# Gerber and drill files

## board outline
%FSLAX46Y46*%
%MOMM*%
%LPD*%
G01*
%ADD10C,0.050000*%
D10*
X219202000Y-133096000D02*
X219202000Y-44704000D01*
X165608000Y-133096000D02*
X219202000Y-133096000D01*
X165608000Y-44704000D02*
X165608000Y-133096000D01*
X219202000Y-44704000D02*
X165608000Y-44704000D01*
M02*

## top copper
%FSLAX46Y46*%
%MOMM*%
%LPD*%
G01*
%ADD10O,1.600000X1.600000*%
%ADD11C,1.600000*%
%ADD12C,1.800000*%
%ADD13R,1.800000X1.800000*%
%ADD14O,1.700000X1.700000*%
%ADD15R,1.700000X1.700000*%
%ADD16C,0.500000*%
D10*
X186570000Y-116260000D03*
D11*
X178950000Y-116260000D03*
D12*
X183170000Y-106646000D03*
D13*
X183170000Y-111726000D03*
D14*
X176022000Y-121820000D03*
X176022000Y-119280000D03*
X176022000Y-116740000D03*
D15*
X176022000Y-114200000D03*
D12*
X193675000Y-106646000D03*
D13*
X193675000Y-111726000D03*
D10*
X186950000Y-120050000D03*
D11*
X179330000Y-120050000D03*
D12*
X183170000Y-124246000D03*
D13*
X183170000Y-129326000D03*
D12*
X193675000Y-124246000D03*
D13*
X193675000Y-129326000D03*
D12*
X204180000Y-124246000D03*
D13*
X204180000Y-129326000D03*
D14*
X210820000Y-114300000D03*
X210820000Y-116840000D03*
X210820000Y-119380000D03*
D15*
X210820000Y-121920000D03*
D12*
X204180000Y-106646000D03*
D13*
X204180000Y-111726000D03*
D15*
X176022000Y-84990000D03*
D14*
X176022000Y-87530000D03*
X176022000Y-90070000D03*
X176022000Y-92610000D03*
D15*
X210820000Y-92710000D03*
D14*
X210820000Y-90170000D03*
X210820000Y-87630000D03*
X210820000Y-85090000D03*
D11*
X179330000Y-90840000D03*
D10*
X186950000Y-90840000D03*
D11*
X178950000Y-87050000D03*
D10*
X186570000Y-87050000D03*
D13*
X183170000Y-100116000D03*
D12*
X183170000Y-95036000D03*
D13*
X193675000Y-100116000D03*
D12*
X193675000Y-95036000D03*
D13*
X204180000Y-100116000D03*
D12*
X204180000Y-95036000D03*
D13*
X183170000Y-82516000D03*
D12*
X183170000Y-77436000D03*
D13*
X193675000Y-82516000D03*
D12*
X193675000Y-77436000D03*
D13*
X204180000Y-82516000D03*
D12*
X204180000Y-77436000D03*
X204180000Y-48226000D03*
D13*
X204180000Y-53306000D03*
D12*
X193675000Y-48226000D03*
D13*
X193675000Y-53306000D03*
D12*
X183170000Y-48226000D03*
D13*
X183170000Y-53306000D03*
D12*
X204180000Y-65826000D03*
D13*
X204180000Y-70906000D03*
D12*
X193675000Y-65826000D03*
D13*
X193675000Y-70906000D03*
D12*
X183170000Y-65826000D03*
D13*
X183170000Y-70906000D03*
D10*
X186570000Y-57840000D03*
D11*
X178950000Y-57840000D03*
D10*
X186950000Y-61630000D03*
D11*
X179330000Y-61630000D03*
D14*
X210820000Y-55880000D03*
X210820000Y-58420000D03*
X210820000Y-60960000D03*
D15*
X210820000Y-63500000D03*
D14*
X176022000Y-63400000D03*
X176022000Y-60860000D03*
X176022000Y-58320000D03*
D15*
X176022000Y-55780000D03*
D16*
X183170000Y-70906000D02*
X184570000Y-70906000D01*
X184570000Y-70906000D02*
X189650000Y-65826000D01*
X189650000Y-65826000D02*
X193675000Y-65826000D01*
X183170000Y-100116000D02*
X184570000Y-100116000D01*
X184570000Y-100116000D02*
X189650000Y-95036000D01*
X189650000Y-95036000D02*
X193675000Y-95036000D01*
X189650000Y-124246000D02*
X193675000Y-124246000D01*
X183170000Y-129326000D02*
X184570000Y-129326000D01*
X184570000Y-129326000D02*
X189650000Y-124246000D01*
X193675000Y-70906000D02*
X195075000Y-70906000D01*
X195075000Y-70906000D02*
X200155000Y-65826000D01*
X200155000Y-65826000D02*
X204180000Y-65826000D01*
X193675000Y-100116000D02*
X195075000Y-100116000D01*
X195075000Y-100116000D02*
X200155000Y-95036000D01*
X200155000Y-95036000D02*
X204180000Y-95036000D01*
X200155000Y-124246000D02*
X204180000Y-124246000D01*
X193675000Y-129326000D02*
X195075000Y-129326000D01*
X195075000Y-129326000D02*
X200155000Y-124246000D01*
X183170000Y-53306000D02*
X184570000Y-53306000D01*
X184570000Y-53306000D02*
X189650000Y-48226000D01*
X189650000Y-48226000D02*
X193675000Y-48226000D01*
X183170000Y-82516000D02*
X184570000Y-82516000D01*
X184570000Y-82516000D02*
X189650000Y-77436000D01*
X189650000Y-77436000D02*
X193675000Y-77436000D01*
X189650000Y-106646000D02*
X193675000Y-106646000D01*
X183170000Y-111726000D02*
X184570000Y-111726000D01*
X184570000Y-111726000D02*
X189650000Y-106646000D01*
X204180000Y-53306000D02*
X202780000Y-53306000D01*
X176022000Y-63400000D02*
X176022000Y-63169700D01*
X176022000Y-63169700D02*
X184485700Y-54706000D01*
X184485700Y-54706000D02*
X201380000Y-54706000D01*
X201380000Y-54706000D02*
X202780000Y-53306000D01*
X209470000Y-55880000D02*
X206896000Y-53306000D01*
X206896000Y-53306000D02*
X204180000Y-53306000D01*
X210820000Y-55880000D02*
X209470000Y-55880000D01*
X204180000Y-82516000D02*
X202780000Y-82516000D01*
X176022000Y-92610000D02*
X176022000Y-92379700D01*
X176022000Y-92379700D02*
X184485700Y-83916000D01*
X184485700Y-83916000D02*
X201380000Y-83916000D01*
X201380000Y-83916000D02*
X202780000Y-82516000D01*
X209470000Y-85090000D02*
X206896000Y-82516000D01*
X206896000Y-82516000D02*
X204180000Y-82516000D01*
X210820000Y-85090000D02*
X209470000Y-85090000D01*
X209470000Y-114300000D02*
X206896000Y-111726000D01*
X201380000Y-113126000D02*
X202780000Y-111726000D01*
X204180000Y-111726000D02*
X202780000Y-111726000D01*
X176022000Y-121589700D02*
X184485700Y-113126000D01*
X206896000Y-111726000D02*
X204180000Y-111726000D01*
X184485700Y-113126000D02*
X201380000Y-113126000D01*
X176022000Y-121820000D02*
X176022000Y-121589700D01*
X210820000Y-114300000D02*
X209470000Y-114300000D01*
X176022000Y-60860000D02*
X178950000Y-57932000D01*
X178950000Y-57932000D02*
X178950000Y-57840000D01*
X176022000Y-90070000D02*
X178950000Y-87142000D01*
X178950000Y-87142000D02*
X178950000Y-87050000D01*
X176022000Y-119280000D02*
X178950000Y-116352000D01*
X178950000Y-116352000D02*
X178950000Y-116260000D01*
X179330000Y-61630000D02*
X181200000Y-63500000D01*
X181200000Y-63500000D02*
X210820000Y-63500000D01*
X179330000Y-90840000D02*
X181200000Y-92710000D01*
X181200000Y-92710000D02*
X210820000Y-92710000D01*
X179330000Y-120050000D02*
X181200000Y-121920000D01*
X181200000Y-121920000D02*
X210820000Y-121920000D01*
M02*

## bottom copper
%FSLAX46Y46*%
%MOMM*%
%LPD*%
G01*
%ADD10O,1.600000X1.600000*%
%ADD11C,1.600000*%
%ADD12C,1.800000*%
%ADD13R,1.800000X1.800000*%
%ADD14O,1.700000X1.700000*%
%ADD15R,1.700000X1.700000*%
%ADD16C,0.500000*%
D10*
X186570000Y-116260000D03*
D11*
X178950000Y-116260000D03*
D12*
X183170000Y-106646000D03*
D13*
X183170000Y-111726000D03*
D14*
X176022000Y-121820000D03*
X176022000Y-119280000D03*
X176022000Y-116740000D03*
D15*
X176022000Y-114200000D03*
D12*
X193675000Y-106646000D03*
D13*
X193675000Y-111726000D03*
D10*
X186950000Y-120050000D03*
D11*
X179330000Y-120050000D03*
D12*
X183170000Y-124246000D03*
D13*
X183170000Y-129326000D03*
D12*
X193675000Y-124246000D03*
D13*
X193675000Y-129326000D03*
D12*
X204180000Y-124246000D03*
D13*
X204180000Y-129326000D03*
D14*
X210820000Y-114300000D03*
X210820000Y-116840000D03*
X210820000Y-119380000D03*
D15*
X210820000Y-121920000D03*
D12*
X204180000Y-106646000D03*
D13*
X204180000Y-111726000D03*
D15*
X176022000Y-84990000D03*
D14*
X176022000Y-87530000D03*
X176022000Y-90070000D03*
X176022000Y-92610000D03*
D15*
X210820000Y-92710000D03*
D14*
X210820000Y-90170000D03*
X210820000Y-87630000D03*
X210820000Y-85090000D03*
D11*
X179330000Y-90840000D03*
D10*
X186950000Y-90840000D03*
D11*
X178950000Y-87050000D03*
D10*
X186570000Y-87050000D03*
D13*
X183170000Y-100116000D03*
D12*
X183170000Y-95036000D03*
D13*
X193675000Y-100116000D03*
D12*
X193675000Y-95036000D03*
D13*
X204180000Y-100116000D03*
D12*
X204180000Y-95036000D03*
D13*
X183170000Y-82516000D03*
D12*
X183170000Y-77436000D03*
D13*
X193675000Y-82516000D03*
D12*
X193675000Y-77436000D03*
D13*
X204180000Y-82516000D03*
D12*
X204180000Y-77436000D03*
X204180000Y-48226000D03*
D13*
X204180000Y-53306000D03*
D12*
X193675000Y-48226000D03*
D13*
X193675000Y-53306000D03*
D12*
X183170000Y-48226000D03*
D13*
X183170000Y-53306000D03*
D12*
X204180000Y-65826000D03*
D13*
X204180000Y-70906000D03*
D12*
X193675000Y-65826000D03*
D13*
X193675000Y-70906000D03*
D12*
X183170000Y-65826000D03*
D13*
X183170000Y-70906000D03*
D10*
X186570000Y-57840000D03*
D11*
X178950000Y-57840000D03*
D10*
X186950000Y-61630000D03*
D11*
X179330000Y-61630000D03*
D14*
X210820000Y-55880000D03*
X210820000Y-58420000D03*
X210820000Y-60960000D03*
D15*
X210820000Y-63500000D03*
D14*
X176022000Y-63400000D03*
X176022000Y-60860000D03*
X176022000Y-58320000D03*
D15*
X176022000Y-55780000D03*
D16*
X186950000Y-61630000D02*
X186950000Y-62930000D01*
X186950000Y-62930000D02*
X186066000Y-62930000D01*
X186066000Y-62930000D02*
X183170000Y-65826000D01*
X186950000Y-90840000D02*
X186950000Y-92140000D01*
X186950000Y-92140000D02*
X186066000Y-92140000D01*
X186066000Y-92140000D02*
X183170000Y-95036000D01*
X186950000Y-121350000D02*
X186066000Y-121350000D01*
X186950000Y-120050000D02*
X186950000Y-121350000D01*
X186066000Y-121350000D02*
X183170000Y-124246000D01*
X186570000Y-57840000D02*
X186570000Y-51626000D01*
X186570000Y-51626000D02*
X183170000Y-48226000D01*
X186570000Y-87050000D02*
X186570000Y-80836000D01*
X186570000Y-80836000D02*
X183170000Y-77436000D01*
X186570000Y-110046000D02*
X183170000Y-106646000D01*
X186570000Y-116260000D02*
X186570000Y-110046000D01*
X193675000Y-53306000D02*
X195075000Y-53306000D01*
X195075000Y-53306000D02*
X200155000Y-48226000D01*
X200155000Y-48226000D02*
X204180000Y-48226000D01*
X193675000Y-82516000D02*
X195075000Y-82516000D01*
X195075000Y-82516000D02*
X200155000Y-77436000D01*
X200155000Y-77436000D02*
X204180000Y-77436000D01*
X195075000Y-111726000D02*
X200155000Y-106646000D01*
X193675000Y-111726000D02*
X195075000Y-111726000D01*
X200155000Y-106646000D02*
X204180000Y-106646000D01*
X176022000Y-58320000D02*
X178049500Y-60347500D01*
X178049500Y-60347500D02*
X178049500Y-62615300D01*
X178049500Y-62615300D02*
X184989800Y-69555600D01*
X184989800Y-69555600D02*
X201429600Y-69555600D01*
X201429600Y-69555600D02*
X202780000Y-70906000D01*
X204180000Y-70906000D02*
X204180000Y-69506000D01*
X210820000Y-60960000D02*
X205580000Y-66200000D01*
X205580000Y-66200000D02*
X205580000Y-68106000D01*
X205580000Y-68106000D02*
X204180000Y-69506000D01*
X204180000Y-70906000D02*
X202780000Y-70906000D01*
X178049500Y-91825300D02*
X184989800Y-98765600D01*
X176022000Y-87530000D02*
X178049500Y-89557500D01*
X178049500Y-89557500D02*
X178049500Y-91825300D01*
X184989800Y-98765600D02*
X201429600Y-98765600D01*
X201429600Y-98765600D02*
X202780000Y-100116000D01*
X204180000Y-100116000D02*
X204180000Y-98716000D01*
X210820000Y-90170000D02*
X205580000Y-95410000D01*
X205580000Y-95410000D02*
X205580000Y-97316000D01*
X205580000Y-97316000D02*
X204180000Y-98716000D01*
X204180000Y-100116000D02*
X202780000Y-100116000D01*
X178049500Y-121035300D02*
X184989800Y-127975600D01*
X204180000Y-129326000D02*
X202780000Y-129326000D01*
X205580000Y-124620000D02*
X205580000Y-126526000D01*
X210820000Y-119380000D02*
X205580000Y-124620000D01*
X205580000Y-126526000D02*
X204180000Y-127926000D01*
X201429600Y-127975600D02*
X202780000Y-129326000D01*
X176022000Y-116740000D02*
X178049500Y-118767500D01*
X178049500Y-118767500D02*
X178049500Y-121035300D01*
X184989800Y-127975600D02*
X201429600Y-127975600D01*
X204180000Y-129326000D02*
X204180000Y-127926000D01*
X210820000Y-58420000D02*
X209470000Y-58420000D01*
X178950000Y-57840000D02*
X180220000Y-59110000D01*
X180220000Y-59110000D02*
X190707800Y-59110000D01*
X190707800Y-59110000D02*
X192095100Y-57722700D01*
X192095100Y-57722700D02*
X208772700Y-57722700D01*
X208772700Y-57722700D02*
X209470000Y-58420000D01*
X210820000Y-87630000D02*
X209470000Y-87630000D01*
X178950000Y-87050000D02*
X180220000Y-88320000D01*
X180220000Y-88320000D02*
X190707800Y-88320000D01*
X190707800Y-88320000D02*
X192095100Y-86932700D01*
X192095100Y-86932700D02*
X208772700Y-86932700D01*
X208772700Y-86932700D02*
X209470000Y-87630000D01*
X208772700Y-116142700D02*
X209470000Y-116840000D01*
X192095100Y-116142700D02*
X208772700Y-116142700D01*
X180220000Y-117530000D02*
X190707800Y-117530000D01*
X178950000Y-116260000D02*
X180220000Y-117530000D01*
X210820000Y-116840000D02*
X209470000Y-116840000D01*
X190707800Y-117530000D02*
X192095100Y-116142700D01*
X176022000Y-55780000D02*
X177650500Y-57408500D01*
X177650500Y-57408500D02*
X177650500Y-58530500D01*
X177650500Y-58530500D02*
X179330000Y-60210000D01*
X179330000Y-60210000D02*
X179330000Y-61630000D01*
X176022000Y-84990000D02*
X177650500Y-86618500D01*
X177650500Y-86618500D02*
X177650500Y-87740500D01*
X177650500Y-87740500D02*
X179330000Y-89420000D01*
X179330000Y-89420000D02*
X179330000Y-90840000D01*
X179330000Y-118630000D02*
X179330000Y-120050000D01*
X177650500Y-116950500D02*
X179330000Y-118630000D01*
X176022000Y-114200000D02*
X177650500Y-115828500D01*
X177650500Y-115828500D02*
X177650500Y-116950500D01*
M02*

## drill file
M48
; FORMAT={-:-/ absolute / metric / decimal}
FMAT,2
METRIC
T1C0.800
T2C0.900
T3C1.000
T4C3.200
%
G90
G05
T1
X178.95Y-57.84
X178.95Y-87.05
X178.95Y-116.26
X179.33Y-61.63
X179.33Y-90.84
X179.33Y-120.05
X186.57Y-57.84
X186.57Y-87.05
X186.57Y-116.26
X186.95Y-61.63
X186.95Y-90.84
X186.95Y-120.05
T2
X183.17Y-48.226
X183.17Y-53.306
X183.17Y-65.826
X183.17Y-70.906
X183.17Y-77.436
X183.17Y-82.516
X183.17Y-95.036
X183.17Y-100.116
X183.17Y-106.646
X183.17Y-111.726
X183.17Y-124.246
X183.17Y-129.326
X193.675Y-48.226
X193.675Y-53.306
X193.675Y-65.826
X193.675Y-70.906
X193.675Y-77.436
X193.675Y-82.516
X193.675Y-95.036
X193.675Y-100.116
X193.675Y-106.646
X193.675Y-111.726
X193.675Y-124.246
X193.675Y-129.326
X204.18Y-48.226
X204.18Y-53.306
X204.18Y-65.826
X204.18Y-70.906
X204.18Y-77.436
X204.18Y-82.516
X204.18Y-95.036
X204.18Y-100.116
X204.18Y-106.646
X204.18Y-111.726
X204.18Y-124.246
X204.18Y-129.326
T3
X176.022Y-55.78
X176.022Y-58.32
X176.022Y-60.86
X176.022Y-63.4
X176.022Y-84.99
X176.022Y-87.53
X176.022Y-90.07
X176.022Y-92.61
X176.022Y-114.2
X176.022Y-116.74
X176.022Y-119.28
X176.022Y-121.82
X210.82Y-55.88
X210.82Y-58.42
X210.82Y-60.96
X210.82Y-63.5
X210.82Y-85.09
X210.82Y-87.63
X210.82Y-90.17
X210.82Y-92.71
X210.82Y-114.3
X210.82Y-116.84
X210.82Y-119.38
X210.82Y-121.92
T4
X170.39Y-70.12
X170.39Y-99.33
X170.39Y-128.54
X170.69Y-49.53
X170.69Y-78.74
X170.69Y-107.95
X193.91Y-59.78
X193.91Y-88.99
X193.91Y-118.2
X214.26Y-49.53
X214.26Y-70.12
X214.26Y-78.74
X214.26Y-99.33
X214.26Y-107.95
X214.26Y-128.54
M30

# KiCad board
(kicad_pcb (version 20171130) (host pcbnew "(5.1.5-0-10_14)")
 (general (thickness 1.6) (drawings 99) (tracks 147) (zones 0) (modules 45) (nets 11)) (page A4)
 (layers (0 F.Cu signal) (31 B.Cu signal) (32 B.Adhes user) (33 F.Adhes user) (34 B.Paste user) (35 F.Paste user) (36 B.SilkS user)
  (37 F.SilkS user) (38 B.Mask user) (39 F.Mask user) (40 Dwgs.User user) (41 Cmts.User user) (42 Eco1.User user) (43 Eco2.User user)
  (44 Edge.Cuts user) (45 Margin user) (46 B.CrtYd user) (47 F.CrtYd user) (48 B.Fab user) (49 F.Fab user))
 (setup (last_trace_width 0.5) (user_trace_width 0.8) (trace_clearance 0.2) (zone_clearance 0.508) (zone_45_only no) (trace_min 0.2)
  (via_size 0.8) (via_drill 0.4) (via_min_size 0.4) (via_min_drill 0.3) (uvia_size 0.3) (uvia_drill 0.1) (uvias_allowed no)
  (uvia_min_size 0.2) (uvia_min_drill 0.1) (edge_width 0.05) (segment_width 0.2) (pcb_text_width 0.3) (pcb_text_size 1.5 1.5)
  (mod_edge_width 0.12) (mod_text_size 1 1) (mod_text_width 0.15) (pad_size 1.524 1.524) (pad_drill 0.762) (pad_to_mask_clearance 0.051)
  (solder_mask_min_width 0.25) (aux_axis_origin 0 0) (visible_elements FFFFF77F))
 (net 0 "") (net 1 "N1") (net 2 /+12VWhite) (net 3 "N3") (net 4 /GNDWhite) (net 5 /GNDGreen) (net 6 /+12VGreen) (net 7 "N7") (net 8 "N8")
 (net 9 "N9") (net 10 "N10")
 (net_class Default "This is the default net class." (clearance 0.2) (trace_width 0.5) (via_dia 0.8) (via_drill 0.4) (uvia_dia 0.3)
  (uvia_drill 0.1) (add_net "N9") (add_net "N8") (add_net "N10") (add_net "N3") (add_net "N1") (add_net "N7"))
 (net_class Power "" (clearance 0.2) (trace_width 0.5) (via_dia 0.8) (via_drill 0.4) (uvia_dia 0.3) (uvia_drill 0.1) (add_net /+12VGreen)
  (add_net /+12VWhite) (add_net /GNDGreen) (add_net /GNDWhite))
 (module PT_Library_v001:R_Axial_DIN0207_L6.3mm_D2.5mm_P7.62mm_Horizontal (layer B.Cu) (at 178.95 116.26)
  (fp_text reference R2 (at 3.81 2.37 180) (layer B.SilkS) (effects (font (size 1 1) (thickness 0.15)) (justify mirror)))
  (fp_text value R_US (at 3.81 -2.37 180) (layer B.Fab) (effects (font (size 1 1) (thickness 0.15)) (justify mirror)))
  (pad 2 thru_hole oval (at 7.62 0) (size 1.6 1.6) (drill 0.8) (layers *.Cu *.Mask) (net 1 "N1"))
  (pad 1 thru_hole circle (at 0 0) (size 1.6 1.6) (drill 0.8) (layers *.Cu *.Mask) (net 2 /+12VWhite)))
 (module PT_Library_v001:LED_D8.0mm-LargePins (layer F.Cu) (at 183.17 111.726 90)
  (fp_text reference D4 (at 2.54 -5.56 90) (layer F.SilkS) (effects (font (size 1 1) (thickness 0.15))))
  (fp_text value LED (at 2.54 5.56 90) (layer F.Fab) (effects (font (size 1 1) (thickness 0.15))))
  (pad 2 thru_hole circle (at 5.08 0 90) (size 1.8 1.8) (drill 0.9) (layers *.Cu *.Mask) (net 1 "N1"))
  (pad 1 thru_hole rect (at 0 0 90) (size 1.8 1.8) (drill 0.9) (layers *.Cu *.Mask) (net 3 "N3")))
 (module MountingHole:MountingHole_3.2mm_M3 (layer F.Cu) (at 214.26 107.95)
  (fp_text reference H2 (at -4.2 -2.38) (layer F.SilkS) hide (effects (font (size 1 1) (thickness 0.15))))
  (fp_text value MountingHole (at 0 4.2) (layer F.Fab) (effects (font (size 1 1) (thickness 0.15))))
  (pad 1 np_thru_hole circle (at 0 0) (size 3.2 3.2) (drill 3.2) (layers *.Cu *.Mask)))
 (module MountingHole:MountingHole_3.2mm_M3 (layer F.Cu) (at 170.39 128.54)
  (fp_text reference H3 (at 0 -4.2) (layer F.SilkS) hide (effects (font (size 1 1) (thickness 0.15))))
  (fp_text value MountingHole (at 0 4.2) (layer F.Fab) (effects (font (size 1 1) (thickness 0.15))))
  (pad 1 np_thru_hole circle (at 0 0) (size 3.2 3.2) (drill 3.2) (layers *.Cu *.Mask)))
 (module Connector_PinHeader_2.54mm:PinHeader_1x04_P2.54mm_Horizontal (layer B.Cu) (at 176.022 114.2 180)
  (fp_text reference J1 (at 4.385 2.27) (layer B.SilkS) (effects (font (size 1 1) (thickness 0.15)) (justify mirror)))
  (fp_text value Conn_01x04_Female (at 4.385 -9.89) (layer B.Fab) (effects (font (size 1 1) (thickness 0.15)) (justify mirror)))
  (pad 4 thru_hole oval (at 0 -7.62 180) (size 1.7 1.7) (drill 1) (layers *.Cu *.Mask) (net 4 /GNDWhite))
  (pad 3 thru_hole oval (at 0 -5.08 180) (size 1.7 1.7) (drill 1) (layers *.Cu *.Mask) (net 2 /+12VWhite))
  (pad 2 thru_hole oval (at 0 -2.54 180) (size 1.7 1.7) (drill 1) (layers *.Cu *.Mask) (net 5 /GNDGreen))
  (pad 1 thru_hole rect (at 0 0 180) (size 1.7 1.7) (drill 1) (layers *.Cu *.Mask) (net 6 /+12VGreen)))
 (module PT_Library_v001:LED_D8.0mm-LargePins (layer F.Cu) (at 193.675 111.726 90)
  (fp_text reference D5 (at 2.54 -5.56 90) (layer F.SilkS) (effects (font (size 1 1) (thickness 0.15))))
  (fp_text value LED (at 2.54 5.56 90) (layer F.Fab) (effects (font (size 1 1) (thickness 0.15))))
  (pad 2 thru_hole circle (at 5.08 0 90) (size 1.8 1.8) (drill 0.9) (layers *.Cu *.Mask) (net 3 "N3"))
  (pad 1 thru_hole rect (at 0 0 90) (size 1.8 1.8) (drill 0.9) (layers *.Cu *.Mask) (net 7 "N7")))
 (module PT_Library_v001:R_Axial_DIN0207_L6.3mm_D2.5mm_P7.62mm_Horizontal (layer B.Cu) (at 179.33 120.05)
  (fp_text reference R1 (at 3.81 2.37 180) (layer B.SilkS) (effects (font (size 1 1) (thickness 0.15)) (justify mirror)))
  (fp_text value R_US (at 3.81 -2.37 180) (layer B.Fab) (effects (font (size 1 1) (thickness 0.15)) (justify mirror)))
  (pad 2 thru_hole oval (at 7.62 0) (size 1.6 1.6) (drill 0.8) (layers *.Cu *.Mask) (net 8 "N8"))
  (pad 1 thru_hole circle (at 0 0) (size 1.6 1.6) (drill 0.8) (layers *.Cu *.Mask) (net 6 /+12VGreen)))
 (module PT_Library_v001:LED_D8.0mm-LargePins (layer F.Cu) (at 183.17 129.326 90)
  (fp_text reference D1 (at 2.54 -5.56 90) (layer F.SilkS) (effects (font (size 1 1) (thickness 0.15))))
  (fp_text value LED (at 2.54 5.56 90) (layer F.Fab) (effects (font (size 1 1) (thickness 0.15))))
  (pad 2 thru_hole circle (at 5.08 0 90) (size 1.8 1.8) (drill 0.9) (layers *.Cu *.Mask) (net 8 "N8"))
  (pad 1 thru_hole rect (at 0 0 90) (size 1.8 1.8) (drill 0.9) (layers *.Cu *.Mask) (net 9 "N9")))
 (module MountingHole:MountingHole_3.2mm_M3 (layer F.Cu) (at 170.69 107.95)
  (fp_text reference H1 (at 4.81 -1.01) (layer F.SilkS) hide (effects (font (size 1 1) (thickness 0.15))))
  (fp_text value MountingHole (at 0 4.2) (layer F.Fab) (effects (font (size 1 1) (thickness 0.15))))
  (pad 1 np_thru_hole circle (at 0 0) (size 3.2 3.2) (drill 3.2) (layers *.Cu *.Mask)))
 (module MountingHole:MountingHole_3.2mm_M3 (layer F.Cu) (at 193.91 118.2)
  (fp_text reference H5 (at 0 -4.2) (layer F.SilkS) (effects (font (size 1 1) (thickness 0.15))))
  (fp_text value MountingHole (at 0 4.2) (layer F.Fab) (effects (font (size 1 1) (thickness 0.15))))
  (pad 1 np_thru_hole circle (at 0 0) (size 3.2 3.2) (drill 3.2) (layers *.Cu *.Mask)))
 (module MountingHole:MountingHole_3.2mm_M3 (layer F.Cu) (at 214.26 128.54)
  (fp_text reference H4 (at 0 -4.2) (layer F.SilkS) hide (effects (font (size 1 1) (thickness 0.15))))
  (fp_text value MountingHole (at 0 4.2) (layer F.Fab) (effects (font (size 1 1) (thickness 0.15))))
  (pad 1 np_thru_hole circle (at 0 0) (size 3.2 3.2) (drill 3.2) (layers *.Cu *.Mask)))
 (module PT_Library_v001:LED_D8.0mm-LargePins (layer F.Cu) (at 193.675 129.326 90)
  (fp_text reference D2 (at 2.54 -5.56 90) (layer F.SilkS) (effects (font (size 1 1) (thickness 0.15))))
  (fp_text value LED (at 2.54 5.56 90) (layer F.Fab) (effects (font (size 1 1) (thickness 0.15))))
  (pad 2 thru_hole circle (at 5.08 0 90) (size 1.8 1.8) (drill 0.9) (layers *.Cu *.Mask) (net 9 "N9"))
  (pad 1 thru_hole rect (at 0 0 90) (size 1.8 1.8) (drill 0.9) (layers *.Cu *.Mask) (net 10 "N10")))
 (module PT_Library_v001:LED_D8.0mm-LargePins (layer F.Cu) (at 204.18 129.326 90)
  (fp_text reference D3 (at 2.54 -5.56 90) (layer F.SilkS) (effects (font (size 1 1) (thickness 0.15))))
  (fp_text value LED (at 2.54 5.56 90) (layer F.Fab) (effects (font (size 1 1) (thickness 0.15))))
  (pad 2 thru_hole circle (at 5.08 0 90) (size 1.8 1.8) (drill 0.9) (layers *.Cu *.Mask) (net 10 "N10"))
  (pad 1 thru_hole rect (at 0 0 90) (size 1.8 1.8) (drill 0.9) (layers *.Cu *.Mask) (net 5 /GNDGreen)))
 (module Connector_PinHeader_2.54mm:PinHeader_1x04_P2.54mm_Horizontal (layer B.Cu) (at 210.82 121.92)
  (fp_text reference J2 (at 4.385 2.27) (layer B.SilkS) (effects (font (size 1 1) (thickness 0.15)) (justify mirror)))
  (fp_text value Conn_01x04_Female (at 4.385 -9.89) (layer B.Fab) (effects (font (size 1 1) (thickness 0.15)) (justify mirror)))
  (pad 4 thru_hole oval (at 0 -7.62) (size 1.7 1.7) (drill 1) (layers *.Cu *.Mask) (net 4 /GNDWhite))
  (pad 3 thru_hole oval (at 0 -5.08) (size 1.7 1.7) (drill 1) (layers *.Cu *.Mask) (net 2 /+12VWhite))
  (pad 2 thru_hole oval (at 0 -2.54) (size 1.7 1.7) (drill 1) (layers *.Cu *.Mask) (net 5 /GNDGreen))
  (pad 1 thru_hole rect (at 0 0) (size 1.7 1.7) (drill 1) (layers *.Cu *.Mask) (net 6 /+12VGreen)))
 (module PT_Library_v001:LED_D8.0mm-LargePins (layer F.Cu) (at 204.18 111.726 90)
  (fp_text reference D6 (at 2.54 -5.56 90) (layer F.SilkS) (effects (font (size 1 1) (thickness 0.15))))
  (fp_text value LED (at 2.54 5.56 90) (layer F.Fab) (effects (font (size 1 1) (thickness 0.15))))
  (pad 2 thru_hole circle (at 5.08 0 90) (size 1.8 1.8) (drill 0.9) (layers *.Cu *.Mask) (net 7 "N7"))
  (pad 1 thru_hole rect (at 0 0 90) (size 1.8 1.8) (drill 0.9) (layers *.Cu *.Mask) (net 4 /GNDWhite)))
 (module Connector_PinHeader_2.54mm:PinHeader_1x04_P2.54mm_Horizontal (layer B.Cu) (at 176.022 84.99 180)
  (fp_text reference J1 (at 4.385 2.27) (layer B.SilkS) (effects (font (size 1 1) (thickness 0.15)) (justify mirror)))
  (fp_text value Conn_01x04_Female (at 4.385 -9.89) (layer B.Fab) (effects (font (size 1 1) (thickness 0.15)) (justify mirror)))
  (pad 1 thru_hole rect (at 0 0 180) (size 1.7 1.7) (drill 1) (layers *.Cu *.Mask) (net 6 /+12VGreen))
  (pad 2 thru_hole oval (at 0 -2.54 180) (size 1.7 1.7) (drill 1) (layers *.Cu *.Mask) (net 5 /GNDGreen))
  (pad 3 thru_hole oval (at 0 -5.08 180) (size 1.7 1.7) (drill 1) (layers *.Cu *.Mask) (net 2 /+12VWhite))
  (pad 4 thru_hole oval (at 0 -7.62 180) (size 1.7 1.7) (drill 1) (layers *.Cu *.Mask) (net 4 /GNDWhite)))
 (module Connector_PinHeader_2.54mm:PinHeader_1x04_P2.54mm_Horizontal (layer B.Cu) (at 210.82 92.71)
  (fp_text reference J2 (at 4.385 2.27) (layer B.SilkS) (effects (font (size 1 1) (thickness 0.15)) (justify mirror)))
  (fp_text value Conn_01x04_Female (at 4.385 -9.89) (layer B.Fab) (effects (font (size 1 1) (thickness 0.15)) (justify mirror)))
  (pad 1 thru_hole rect (at 0 0) (size 1.7 1.7) (drill 1) (layers *.Cu *.Mask) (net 6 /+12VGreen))
  (pad 2 thru_hole oval (at 0 -2.54) (size 1.7 1.7) (drill 1) (layers *.Cu *.Mask) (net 5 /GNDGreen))
  (pad 3 thru_hole oval (at 0 -5.08) (size 1.7 1.7) (drill 1) (layers *.Cu *.Mask) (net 2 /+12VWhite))
  (pad 4 thru_hole oval (at 0 -7.62) (size 1.7 1.7) (drill 1) (layers *.Cu *.Mask) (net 4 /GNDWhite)))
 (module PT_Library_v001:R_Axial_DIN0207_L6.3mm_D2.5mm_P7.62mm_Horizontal (layer B.Cu) (at 179.33 90.84)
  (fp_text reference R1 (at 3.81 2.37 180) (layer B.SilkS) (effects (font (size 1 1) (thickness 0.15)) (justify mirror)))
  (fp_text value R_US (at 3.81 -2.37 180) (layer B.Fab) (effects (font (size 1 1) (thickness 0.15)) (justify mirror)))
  (pad 1 thru_hole circle (at 0 0) (size 1.6 1.6) (drill 0.8) (layers *.Cu *.Mask) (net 6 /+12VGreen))
  (pad 2 thru_hole oval (at 7.62 0) (size 1.6 1.6) (drill 0.8) (layers *.Cu *.Mask) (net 8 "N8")))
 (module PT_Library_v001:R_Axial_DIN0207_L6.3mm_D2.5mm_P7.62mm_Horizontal (layer B.Cu) (at 178.95 87.05)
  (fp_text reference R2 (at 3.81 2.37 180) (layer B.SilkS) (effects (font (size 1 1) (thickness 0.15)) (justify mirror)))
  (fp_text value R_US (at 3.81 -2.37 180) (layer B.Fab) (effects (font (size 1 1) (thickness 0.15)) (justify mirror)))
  (pad 1 thru_hole circle (at 0 0) (size 1.6 1.6) (drill 0.8) (layers *.Cu *.Mask) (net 2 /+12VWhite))
  (pad 2 thru_hole oval (at 7.62 0) (size 1.6 1.6) (drill 0.8) (layers *.Cu *.Mask) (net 1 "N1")))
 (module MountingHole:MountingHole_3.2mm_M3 (layer F.Cu) (at 170.69 78.74)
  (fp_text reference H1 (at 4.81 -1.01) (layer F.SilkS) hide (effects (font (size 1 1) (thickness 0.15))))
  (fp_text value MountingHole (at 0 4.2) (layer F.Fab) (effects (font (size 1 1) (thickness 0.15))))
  (pad 1 np_thru_hole circle (at 0 0) (size 3.2 3.2) (drill 3.2) (layers *.Cu *.Mask)))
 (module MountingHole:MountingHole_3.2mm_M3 (layer F.Cu) (at 214.26 78.74)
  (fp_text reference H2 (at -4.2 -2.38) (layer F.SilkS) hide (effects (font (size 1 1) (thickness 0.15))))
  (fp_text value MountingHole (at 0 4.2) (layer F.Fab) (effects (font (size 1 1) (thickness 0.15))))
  (pad 1 np_thru_hole circle (at 0 0) (size 3.2 3.2) (drill 3.2) (layers *.Cu *.Mask)))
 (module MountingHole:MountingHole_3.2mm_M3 (layer F.Cu) (at 170.39 99.33)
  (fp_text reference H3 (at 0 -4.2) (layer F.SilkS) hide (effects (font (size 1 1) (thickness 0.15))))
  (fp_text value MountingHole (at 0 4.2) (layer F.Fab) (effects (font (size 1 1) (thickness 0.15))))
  (pad 1 np_thru_hole circle (at 0 0) (size 3.2 3.2) (drill 3.2) (layers *.Cu *.Mask)))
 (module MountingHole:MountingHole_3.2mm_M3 (layer F.Cu) (at 214.26 99.33)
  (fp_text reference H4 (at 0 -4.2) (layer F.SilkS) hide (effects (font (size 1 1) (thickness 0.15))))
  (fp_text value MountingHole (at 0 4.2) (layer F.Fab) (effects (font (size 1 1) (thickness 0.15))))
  (pad 1 np_thru_hole circle (at 0 0) (size 3.2 3.2) (drill 3.2) (layers *.Cu *.Mask)))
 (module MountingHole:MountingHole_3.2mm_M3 (layer F.Cu) (at 193.91 88.99)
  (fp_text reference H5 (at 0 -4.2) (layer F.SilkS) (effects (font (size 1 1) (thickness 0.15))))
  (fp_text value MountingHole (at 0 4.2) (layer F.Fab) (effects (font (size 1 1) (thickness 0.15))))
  (pad 1 np_thru_hole circle (at 0 0) (size 3.2 3.2) (drill 3.2) (layers *.Cu *.Mask)))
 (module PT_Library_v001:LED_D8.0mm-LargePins (layer F.Cu) (at 183.17 100.116 90)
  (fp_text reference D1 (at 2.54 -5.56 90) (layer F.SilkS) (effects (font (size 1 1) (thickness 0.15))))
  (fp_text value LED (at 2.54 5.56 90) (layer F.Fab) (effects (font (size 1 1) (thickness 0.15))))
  (pad 1 thru_hole rect (at 0 0 90) (size 1.8 1.8) (drill 0.9) (layers *.Cu *.Mask) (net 9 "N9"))
  (pad 2 thru_hole circle (at 5.08 0 90) (size 1.8 1.8) (drill 0.9) (layers *.Cu *.Mask) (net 8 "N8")))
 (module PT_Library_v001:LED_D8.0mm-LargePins (layer F.Cu) (at 193.675 100.116 90)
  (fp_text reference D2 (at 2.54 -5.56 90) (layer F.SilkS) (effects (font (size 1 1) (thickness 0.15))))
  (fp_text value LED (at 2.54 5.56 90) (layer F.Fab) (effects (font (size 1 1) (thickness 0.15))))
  (pad 1 thru_hole rect (at 0 0 90) (size 1.8 1.8) (drill 0.9) (layers *.Cu *.Mask) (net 10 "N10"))
  (pad 2 thru_hole circle (at 5.08 0 90) (size 1.8 1.8) (drill 0.9) (layers *.Cu *.Mask) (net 9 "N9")))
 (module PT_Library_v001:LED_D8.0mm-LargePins (layer F.Cu) (at 204.18 100.116 90)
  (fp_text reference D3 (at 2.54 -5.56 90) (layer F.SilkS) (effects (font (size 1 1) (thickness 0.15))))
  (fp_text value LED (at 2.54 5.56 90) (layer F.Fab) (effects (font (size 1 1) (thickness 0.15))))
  (pad 1 thru_hole rect (at 0 0 90) (size 1.8 1.8) (drill 0.9) (layers *.Cu *.Mask) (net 5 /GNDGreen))
  (pad 2 thru_hole circle (at 5.08 0 90) (size 1.8 1.8) (drill 0.9) (layers *.Cu *.Mask) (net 10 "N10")))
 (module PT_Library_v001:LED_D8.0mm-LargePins (layer F.Cu) (at 183.17 82.516 90)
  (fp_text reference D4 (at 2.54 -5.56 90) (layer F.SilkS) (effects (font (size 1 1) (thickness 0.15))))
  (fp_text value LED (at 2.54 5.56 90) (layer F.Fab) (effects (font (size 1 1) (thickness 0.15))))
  (pad 1 thru_hole rect (at 0 0 90) (size 1.8 1.8) (drill 0.9) (layers *.Cu *.Mask) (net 3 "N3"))
  (pad 2 thru_hole circle (at 5.08 0 90) (size 1.8 1.8) (drill 0.9) (layers *.Cu *.Mask) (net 1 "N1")))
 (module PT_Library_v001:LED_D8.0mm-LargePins (layer F.Cu) (at 193.675 82.516 90)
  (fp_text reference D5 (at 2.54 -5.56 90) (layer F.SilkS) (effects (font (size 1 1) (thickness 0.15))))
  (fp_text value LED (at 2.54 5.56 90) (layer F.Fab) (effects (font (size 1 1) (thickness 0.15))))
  (pad 1 thru_hole rect (at 0 0 90) (size 1.8 1.8) (drill 0.9) (layers *.Cu *.Mask) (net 7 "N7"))
  (pad 2 thru_hole circle (at 5.08 0 90) (size 1.8 1.8) (drill 0.9) (layers *.Cu *.Mask) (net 3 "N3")))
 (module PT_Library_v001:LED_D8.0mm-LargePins (layer F.Cu) (at 204.18 82.516 90)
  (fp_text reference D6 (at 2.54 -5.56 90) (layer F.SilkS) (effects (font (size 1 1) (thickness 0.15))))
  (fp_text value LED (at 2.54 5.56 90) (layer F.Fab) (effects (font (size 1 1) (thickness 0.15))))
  (pad 1 thru_hole rect (at 0 0 90) (size 1.8 1.8) (drill 0.9) (layers *.Cu *.Mask) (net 4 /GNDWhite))
  (pad 2 thru_hole circle (at 5.08 0 90) (size 1.8 1.8) (drill 0.9) (layers *.Cu *.Mask) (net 7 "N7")))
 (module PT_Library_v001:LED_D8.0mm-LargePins (layer F.Cu) (at 204.18 53.306 90)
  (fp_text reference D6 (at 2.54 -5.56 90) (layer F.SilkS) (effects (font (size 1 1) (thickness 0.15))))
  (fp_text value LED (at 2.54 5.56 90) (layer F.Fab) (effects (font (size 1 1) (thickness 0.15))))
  (pad 2 thru_hole circle (at 5.08 0 90) (size 1.8 1.8) (drill 0.9) (layers *.Cu *.Mask) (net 7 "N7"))
  (pad 1 thru_hole rect (at 0 0 90) (size 1.8 1.8) (drill 0.9) (layers *.Cu *.Mask) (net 4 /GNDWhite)))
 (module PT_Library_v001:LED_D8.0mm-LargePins (layer F.Cu) (at 193.675 53.306 90)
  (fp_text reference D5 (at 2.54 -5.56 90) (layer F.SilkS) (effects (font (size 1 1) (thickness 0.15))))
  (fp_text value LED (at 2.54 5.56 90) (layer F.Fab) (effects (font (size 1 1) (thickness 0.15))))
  (pad 2 thru_hole circle (at 5.08 0 90) (size 1.8 1.8) (drill 0.9) (layers *.Cu *.Mask) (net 3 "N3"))
  (pad 1 thru_hole rect (at 0 0 90) (size 1.8 1.8) (drill 0.9) (layers *.Cu *.Mask) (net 7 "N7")))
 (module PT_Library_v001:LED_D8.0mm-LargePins (layer F.Cu) (at 183.17 53.306 90)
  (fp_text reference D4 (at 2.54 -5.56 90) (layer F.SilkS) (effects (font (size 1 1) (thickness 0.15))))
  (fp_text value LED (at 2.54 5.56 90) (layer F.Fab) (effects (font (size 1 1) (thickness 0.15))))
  (pad 2 thru_hole circle (at 5.08 0 90) (size 1.8 1.8) (drill 0.9) (layers *.Cu *.Mask) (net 1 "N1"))
  (pad 1 thru_hole rect (at 0 0 90) (size 1.8 1.8) (drill 0.9) (layers *.Cu *.Mask) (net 3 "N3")))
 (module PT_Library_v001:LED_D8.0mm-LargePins (layer F.Cu) (at 204.18 70.906 90)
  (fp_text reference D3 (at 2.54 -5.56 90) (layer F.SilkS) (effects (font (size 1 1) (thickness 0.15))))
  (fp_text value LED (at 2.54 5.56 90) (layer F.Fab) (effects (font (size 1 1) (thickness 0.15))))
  (pad 2 thru_hole circle (at 5.08 0 90) (size 1.8 1.8) (drill 0.9) (layers *.Cu *.Mask) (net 10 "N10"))
  (pad 1 thru_hole rect (at 0 0 90) (size 1.8 1.8) (drill 0.9) (layers *.Cu *.Mask) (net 5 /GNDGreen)))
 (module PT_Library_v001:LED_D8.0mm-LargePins (layer F.Cu) (at 193.675 70.906 90)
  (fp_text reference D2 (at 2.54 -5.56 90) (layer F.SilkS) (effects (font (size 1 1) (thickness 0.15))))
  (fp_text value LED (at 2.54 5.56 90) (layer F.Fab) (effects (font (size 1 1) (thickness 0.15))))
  (pad 2 thru_hole circle (at 5.08 0 90) (size 1.8 1.8) (drill 0.9) (layers *.Cu *.Mask) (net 9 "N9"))
  (pad 1 thru_hole rect (at 0 0 90) (size 1.8 1.8) (drill 0.9) (layers *.Cu *.Mask) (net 10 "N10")))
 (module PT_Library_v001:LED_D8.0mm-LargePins (layer F.Cu) (at 183.17 70.906 90)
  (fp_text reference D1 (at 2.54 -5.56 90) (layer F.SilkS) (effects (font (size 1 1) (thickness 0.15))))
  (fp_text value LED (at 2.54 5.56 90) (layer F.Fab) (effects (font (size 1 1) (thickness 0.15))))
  (pad 2 thru_hole circle (at 5.08 0 90) (size 1.8 1.8) (drill 0.9) (layers *.Cu *.Mask) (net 8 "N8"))
  (pad 1 thru_hole rect (at 0 0 90) (size 1.8 1.8) (drill 0.9) (layers *.Cu *.Mask) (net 9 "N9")))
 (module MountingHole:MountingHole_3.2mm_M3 (layer F.Cu) (at 193.91 59.78)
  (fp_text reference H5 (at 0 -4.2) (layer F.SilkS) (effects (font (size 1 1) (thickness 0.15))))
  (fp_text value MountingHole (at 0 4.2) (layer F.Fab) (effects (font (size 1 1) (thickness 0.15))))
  (pad 1 np_thru_hole circle (at 0 0) (size 3.2 3.2) (drill 3.2) (layers *.Cu *.Mask)))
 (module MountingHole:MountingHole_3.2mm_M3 (layer F.Cu) (at 214.26 70.12)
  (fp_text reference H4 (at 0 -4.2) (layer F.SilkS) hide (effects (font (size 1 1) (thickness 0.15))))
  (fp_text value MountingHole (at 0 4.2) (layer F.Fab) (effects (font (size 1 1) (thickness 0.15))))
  (pad 1 np_thru_hole circle (at 0 0) (size 3.2 3.2) (drill 3.2) (layers *.Cu *.Mask)))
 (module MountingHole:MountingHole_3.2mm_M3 (layer F.Cu) (at 170.39 70.12)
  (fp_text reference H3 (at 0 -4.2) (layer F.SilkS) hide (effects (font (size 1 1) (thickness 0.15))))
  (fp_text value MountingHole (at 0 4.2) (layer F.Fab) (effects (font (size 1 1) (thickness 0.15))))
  (pad 1 np_thru_hole circle (at 0 0) (size 3.2 3.2) (drill 3.2) (layers *.Cu *.Mask)))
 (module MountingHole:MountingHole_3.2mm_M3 (layer F.Cu) (at 214.26 49.53)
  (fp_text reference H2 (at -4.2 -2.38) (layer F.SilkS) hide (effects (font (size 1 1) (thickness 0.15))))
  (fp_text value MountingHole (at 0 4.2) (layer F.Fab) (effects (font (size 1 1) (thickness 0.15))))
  (pad 1 np_thru_hole circle (at 0 0) (size 3.2 3.2) (drill 3.2) (layers *.Cu *.Mask)))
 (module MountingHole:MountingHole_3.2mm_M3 (layer F.Cu) (at 170.69 49.53)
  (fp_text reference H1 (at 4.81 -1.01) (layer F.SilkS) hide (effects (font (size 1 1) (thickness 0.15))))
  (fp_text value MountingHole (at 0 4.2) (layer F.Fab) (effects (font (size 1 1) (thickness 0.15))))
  (pad 1 np_thru_hole circle (at 0 0) (size 3.2 3.2) (drill 3.2) (layers *.Cu *.Mask)))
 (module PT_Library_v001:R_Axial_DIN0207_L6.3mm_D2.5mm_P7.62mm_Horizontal (layer B.Cu) (at 178.95 57.84)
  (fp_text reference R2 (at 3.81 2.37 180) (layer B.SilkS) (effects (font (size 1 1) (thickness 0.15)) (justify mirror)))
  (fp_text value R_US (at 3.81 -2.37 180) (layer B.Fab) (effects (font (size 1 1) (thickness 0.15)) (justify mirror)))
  (pad 2 thru_hole oval (at 7.62 0) (size 1.6 1.6) (drill 0.8) (layers *.Cu *.Mask) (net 1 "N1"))
  (pad 1 thru_hole circle (at 0 0) (size 1.6 1.6) (drill 0.8) (layers *.Cu *.Mask) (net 2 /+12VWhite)))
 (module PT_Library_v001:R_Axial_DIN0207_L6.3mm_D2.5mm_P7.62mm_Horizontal (layer B.Cu) (at 179.33 61.63)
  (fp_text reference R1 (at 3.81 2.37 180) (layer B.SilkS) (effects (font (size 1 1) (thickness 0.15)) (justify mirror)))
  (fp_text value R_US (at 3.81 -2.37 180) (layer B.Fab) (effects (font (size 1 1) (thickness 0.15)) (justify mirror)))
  (pad 2 thru_hole oval (at 7.62 0) (size 1.6 1.6) (drill 0.8) (layers *.Cu *.Mask) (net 8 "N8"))
  (pad 1 thru_hole circle (at 0 0) (size 1.6 1.6) (drill 0.8) (layers *.Cu *.Mask) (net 6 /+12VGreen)))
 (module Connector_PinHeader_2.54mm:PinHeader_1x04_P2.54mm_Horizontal (layer B.Cu) (at 210.82 63.5)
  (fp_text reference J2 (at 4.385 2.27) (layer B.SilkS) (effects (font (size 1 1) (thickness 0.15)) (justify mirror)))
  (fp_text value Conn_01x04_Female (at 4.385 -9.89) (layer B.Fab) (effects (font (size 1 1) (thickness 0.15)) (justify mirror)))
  (pad 4 thru_hole oval (at 0 -7.62) (size 1.7 1.7) (drill 1) (layers *.Cu *.Mask) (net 4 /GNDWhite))
  (pad 3 thru_hole oval (at 0 -5.08) (size 1.7 1.7) (drill 1) (layers *.Cu *.Mask) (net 2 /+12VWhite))
  (pad 2 thru_hole oval (at 0 -2.54) (size 1.7 1.7) (drill 1) (layers *.Cu *.Mask) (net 5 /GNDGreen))
  (pad 1 thru_hole rect (at 0 0) (size 1.7 1.7) (drill 1) (layers *.Cu *.Mask) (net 6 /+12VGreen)))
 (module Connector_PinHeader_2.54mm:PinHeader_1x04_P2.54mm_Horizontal (layer B.Cu) (at 176.022 55.78 180)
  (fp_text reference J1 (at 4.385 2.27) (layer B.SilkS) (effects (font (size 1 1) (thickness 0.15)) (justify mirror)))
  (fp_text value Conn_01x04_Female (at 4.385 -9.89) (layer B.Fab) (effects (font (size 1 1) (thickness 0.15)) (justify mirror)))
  (pad 4 thru_hole oval (at 0 -7.62 180) (size 1.7 1.7) (drill 1) (layers *.Cu *.Mask) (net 4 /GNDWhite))
  (pad 3 thru_hole oval (at 0 -5.08 180) (size 1.7 1.7) (drill 1) (layers *.Cu *.Mask) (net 2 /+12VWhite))
  (pad 2 thru_hole oval (at 0 -2.54 180) (size 1.7 1.7) (drill 1) (layers *.Cu *.Mask) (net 5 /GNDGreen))
  (pad 1 thru_hole rect (at 0 0 180) (size 1.7 1.7) (drill 1) (layers *.Cu *.Mask) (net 6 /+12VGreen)))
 (gr_line (start 219.202 133.096) (end 219.202 44.704) (layer Edge.Cuts) (width 0.05))
 (gr_line (start 165.608 133.096) (end 219.202 133.096) (layer Edge.Cuts) (width 0.05))
 (gr_line (start 165.608 44.704) (end 165.608 133.096) (layer Edge.Cuts) (width 0.05))
 (gr_line (start 219.202 44.704) (end 165.608 44.704) (layer Edge.Cuts) (width 0.05))
 (segment (start 183.17 70.906) (end 184.57 70.906) (width 0.5) (layer F.Cu) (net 9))
 (segment (start 184.57 70.906) (end 189.65 65.826) (width 0.5) (layer F.Cu) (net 9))
 (segment (start 189.65 65.826) (end 193.675 65.826) (width 0.5) (layer F.Cu) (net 9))
 (segment (start 183.17 100.116) (end 184.57 100.116) (width 0.5) (layer F.Cu) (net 9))
 (segment (start 184.57 100.116) (end 189.65 95.036) (width 0.5) (layer F.Cu) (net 9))
 (segment (start 189.65 95.036) (end 193.675 95.036) (width 0.5) (layer F.Cu) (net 9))
 (segment (start 189.65 124.246) (end 193.675 124.246) (width 0.5) (layer F.Cu) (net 9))
 (segment (start 183.17 129.326) (end 184.57 129.326) (width 0.5) (layer F.Cu) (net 9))
 (segment (start 184.57 129.326) (end 189.65 124.246) (width 0.5) (layer F.Cu) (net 9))
 (segment (start 186.95 61.63) (end 186.95 62.93) (width 0.5) (layer B.Cu) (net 8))
 (segment (start 186.95 62.93) (end 186.066 62.93) (width 0.5) (layer B.Cu) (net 8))
 (segment (start 186.066 62.93) (end 183.17 65.826) (width 0.5) (layer B.Cu) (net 8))
 (segment (start 186.95 90.84) (end 186.95 92.14) (width 0.5) (layer B.Cu) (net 8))
 (segment (start 186.95 92.14) (end 186.066 92.14) (width 0.5) (layer B.Cu) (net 8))
 (segment (start 186.066 92.14) (end 183.17 95.036) (width 0.5) (layer B.Cu) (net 8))
 (segment (start 186.95 121.35) (end 186.066 121.35) (width 0.5) (layer B.Cu) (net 8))
 (segment (start 186.95 120.05) (end 186.95 121.35) (width 0.5) (layer B.Cu) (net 8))
 (segment (start 186.066 121.35) (end 183.17 124.246) (width 0.5) (layer B.Cu) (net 8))
 (segment (start 193.675 70.906) (end 195.075 70.906) (width 0.5) (layer F.Cu) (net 10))
 (segment (start 195.075 70.906) (end 200.155 65.826) (width 0.5) (layer F.Cu) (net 10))
 (segment (start 200.155 65.826) (end 204.18 65.826) (width 0.5) (layer F.Cu) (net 10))
 (segment (start 193.675 100.116) (end 195.075 100.116) (width 0.5) (layer F.Cu) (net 10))
 (segment (start 195.075 100.116) (end 200.155 95.036) (width 0.5) (layer F.Cu) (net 10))
 (segment (start 200.155 95.036) (end 204.18 95.036) (width 0.5) (layer F.Cu) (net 10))
 (segment (start 200.155 124.246) (end 204.18 124.246) (width 0.5) (layer F.Cu) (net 10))
 (segment (start 193.675 129.326) (end 195.075 129.326) (width 0.5) (layer F.Cu) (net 10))
 (segment (start 195.075 129.326) (end 200.155 124.246) (width 0.5) (layer F.Cu) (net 10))
 (segment (start 186.57 57.84) (end 186.57 51.626) (width 0.5) (layer B.Cu) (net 1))
 (segment (start 186.57 51.626) (end 183.17 48.226) (width 0.5) (layer B.Cu) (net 1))
 (segment (start 186.57 87.05) (end 186.57 80.836) (width 0.5) (layer B.Cu) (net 1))
 (segment (start 186.57 80.836) (end 183.17 77.436) (width 0.5) (layer B.Cu) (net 1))
 (segment (start 186.57 110.046) (end 183.17 106.646) (width 0.5) (layer B.Cu) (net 1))
 (segment (start 186.57 116.26) (end 186.57 110.046) (width 0.5) (layer B.Cu) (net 1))
 (segment (start 183.17 53.306) (end 184.57 53.306) (width 0.5) (layer F.Cu) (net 3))
 (segment (start 184.57 53.306) (end 189.65 48.226) (width 0.5) (layer F.Cu) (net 3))
 (segment (start 189.65 48.226) (end 193.675 48.226) (width 0.5) (layer F.Cu) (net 3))
 (segment (start 183.17 82.516) (end 184.57 82.516) (width 0.5) (layer F.Cu) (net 3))
 (segment (start 184.57 82.516) (end 189.65 77.436) (width 0.5) (layer F.Cu) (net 3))
 (segment (start 189.65 77.436) (end 193.675 77.436) (width 0.5) (layer F.Cu) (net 3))
 (segment (start 189.65 106.646) (end 193.675 106.646) (width 0.5) (layer F.Cu) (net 3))
 (segment (start 183.17 111.726) (end 184.57 111.726) (width 0.5) (layer F.Cu) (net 3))
 (segment (start 184.57 111.726) (end 189.65 106.646) (width 0.5) (layer F.Cu) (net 3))
 (segment (start 193.675 53.306) (end 195.075 53.306) (width 0.5) (layer B.Cu) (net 7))
 (segment (start 195.075 53.306) (end 200.155 48.226) (width 0.5) (layer B.Cu) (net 7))
 (segment (start 200.155 48.226) (end 204.18 48.226) (width 0.5) (layer B.Cu) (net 7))
 (segment (start 193.675 82.516) (end 195.075 82.516) (width 0.5) (layer B.Cu) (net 7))
 (segment (start 195.075 82.516) (end 200.155 77.436) (width 0.5) (layer B.Cu) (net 7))
 (segment (start 200.155 77.436) (end 204.18 77.436) (width 0.5) (layer B.Cu) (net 7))
 (segment (start 195.075 111.726) (end 200.155 106.646) (width 0.5) (layer B.Cu) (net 7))
 (segment (start 193.675 111.726) (end 195.075 111.726) (width 0.5) (layer B.Cu) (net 7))
 (segment (start 200.155 106.646) (end 204.18 106.646) (width 0.5) (layer B.Cu) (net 7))
 (segment (start 176.022 58.32) (end 178.0495 60.3475) (width 0.5) (layer B.Cu) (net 5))
 (segment (start 178.0495 60.3475) (end 178.0495 62.6153) (width 0.5) (layer B.Cu) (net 5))
 (segment (start 178.0495 62.6153) (end 184.9898 69.5556) (width 0.5) (layer B.Cu) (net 5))
 (segment (start 184.9898 69.5556) (end 201.4296 69.5556) (width 0.5) (layer B.Cu) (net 5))
 (segment (start 201.4296 69.5556) (end 202.78 70.906) (width 0.5) (layer B.Cu) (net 5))
 (segment (start 204.18 70.906) (end 204.18 69.506) (width 0.5) (layer B.Cu) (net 5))
 (segment (start 210.82 60.96) (end 205.58 66.2) (width 0.5) (layer B.Cu) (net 5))
 (segment (start 205.58 66.2) (end 205.58 68.106) (width 0.5) (layer B.Cu) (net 5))
 (segment (start 205.58 68.106) (end 204.18 69.506) (width 0.5) (layer B.Cu) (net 5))
 (segment (start 204.18 70.906) (end 202.78 70.906) (width 0.5) (layer B.Cu) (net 5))
 (segment (start 178.0495 91.8253) (end 184.9898 98.7656) (width 0.5) (layer B.Cu) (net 5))
 (segment (start 176.022 87.53) (end 178.0495 89.5575) (width 0.5) (layer B.Cu) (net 5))
 (segment (start 178.0495 89.5575) (end 178.0495 91.8253) (width 0.5) (layer B.Cu) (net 5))
 (segment (start 184.9898 98.7656) (end 201.4296 98.7656) (width 0.5) (layer B.Cu) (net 5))
 (segment (start 201.4296 98.7656) (end 202.78 100.116) (width 0.5) (layer B.Cu) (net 5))
 (segment (start 204.18 100.116) (end 204.18 98.716) (width 0.5) (layer B.Cu) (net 5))
 (segment (start 210.82 90.17) (end 205.58 95.41) (width 0.5) (layer B.Cu) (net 5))
 (segment (start 205.58 95.41) (end 205.58 97.316) (width 0.5) (layer B.Cu) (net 5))
 (segment (start 205.58 97.316) (end 204.18 98.716) (width 0.5) (layer B.Cu) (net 5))
 (segment (start 204.18 100.116) (end 202.78 100.116) (width 0.5) (layer B.Cu) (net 5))
 (segment (start 178.0495 121.0353) (end 184.9898 127.9756) (width 0.5) (layer B.Cu) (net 5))
 (segment (start 204.18 129.326) (end 202.78 129.326) (width 0.5) (layer B.Cu) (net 5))
 (segment (start 205.58 124.62) (end 205.58 126.526) (width 0.5) (layer B.Cu) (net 5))
 (segment (start 210.82 119.38) (end 205.58 124.62) (width 0.5) (layer B.Cu) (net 5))
 (segment (start 205.58 126.526) (end 204.18 127.926) (width 0.5) (layer B.Cu) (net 5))
 (segment (start 201.4296 127.9756) (end 202.78 129.326) (width 0.5) (layer B.Cu) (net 5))
 (segment (start 176.022 116.74) (end 178.0495 118.7675) (width 0.5) (layer B.Cu) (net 5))
 (segment (start 178.0495 118.7675) (end 178.0495 121.0353) (width 0.5) (layer B.Cu) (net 5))
 (segment (start 184.9898 127.9756) (end 201.4296 127.9756) (width 0.5) (layer B.Cu) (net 5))
 (segment (start 204.18 129.326) (end 204.18 127.926) (width 0.5) (layer B.Cu) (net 5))
 (segment (start 204.18 53.306) (end 202.78 53.306) (width 0.5) (layer F.Cu) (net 4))
 (segment (start 176.022 63.4) (end 176.022 63.1697) (width 0.5) (layer F.Cu) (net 4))
 (segment (start 176.022 63.1697) (end 184.4857 54.706) (width 0.5) (layer F.Cu) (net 4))
 (segment (start 184.4857 54.706) (end 201.38 54.706) (width 0.5) (layer F.Cu) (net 4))
 (segment (start 201.38 54.706) (end 202.78 53.306) (width 0.5) (layer F.Cu) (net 4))
 (segment (start 209.47 55.88) (end 206.896 53.306) (width 0.5) (layer F.Cu) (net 4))
 (segment (start 206.896 53.306) (end 204.18 53.306) (width 0.5) (layer F.Cu) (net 4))
 (segment (start 210.82 55.88) (end 209.47 55.88) (width 0.5) (layer F.Cu) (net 4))
 (segment (start 204.18 82.516) (end 202.78 82.516) (width 0.5) (layer F.Cu) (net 4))
 (segment (start 176.022 92.61) (end 176.022 92.3797) (width 0.5) (layer F.Cu) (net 4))
 (segment (start 176.022 92.3797) (end 184.4857 83.916) (width 0.5) (layer F.Cu) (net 4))
 (segment (start 184.4857 83.916) (end 201.38 83.916) (width 0.5) (layer F.Cu) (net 4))
 (segment (start 201.38 83.916) (end 202.78 82.516) (width 0.5) (layer F.Cu) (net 4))
 (segment (start 209.47 85.09) (end 206.896 82.516) (width 0.5) (layer F.Cu) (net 4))
 (segment (start 206.896 82.516) (end 204.18 82.516) (width 0.5) (layer F.Cu) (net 4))
 (segment (start 210.82 85.09) (end 209.47 85.09) (width 0.5) (layer F.Cu) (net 4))
 (segment (start 209.47 114.3) (end 206.896 111.726) (width 0.5) (layer F.Cu) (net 4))
 (segment (start 201.38 113.126) (end 202.78 111.726) (width 0.5) (layer F.Cu) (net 4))
 (segment (start 204.18 111.726) (end 202.78 111.726) (width 0.5) (layer F.Cu) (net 4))
 (segment (start 176.022 121.5897) (end 184.4857 113.126) (width 0.5) (layer F.Cu) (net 4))
 (segment (start 206.896 111.726) (end 204.18 111.726) (width 0.5) (layer F.Cu) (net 4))
 (segment (start 184.4857 113.126) (end 201.38 113.126) (width 0.5) (layer F.Cu) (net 4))
 (segment (start 176.022 121.82) (end 176.022 121.5897) (width 0.5) (layer F.Cu) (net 4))
 (segment (start 210.82 114.3) (end 209.47 114.3) (width 0.5) (layer F.Cu) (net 4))
 (segment (start 210.82 58.42) (end 209.47 58.42) (width 0.5) (layer B.Cu) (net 2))
 (segment (start 178.95 57.84) (end 180.22 59.11) (width 0.5) (layer B.Cu) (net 2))
 (segment (start 180.22 59.11) (end 190.7078 59.11) (width 0.5) (layer B.Cu) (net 2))
 (segment (start 190.7078 59.11) (end 192.0951 57.7227) (width 0.5) (layer B.Cu) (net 2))
 (segment (start 192.0951 57.7227) (end 208.7727 57.7227) (width 0.5) (layer B.Cu) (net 2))
 (segment (start 208.7727 57.7227) (end 209.47 58.42) (width 0.5) (layer B.Cu) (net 2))
 (segment (start 176.022 60.86) (end 178.95 57.932) (width 0.5) (layer F.Cu) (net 2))
 (segment (start 178.95 57.932) (end 178.95 57.84) (width 0.5) (layer F.Cu) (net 2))
 (segment (start 210.82 87.63) (end 209.47 87.63) (width 0.5) (layer B.Cu) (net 2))
 (segment (start 178.95 87.05) (end 180.22 88.32) (width 0.5) (layer B.Cu) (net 2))
 (segment (start 180.22 88.32) (end 190.7078 88.32) (width 0.5) (layer B.Cu) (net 2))
 (segment (start 190.7078 88.32) (end 192.0951 86.9327) (width 0.5) (layer B.Cu) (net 2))
 (segment (start 192.0951 86.9327) (end 208.7727 86.9327) (width 0.5) (layer B.Cu) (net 2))
 (segment (start 208.7727 86.9327) (end 209.47 87.63) (width 0.5) (layer B.Cu) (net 2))
 (segment (start 176.022 90.07) (end 178.95 87.142) (width 0.5) (layer F.Cu) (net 2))
 (segment (start 178.95 87.142) (end 178.95 87.05) (width 0.5) (layer F.Cu) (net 2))
 (segment (start 176.022 119.28) (end 178.95 116.352) (width 0.5) (layer F.Cu) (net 2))
 (segment (start 178.95 116.352) (end 178.95 116.26) (width 0.5) (layer F.Cu) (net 2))
 (segment (start 208.7727 116.1427) (end 209.47 116.84) (width 0.5) (layer B.Cu) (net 2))
 (segment (start 192.0951 116.1427) (end 208.7727 116.1427) (width 0.5) (layer B.Cu) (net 2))
 (segment (start 180.22 117.53) (end 190.7078 117.53) (width 0.5) (layer B.Cu) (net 2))
 (segment (start 178.95 116.26) (end 180.22 117.53) (width 0.5) (layer B.Cu) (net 2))
 (segment (start 210.82 116.84) (end 209.47 116.84) (width 0.5) (layer B.Cu) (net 2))
 (segment (start 190.7078 117.53) (end 192.0951 116.1427) (width 0.5) (layer B.Cu) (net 2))
 (segment (start 176.022 55.78) (end 177.6505 57.4085) (width 0.5) (layer B.Cu) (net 6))
 (segment (start 177.6505 57.4085) (end 177.6505 58.5305) (width 0.5) (layer B.Cu) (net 6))
 (segment (start 177.6505 58.5305) (end 179.33 60.21) (width 0.5) (layer B.Cu) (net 6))
 (segment (start 179.33 60.21) (end 179.33 61.63) (width 0.5) (layer B.Cu) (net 6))
 (segment (start 179.33 61.63) (end 181.2 63.5) (width 0.5) (layer F.Cu) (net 6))
 (segment (start 181.2 63.5) (end 210.82 63.5) (width 0.5) (layer F.Cu) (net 6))
 (segment (start 176.022 84.99) (end 177.6505 86.6185) (width 0.5) (layer B.Cu) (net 6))
 (segment (start 177.6505 86.6185) (end 177.6505 87.7405) (width 0.5) (layer B.Cu) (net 6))
 (segment (start 177.6505 87.7405) (end 179.33 89.42) (width 0.5) (layer B.Cu) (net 6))
 (segment (start 179.33 89.42) (end 179.33 90.84) (width 0.5) (layer B.Cu) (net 6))
 (segment (start 179.33 90.84) (end 181.2 92.71) (width 0.5) (layer F.Cu) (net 6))
 (segment (start 181.2 92.71) (end 210.82 92.71) (width 0.5) (layer F.Cu) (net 6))
 (segment (start 179.33 118.63) (end 179.33 120.05) (width 0.5) (layer B.Cu) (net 6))
 (segment (start 177.6505 116.9505) (end 179.33 118.63) (width 0.5) (layer B.Cu) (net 6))
 (segment (start 179.33 120.05) (end 181.2 121.92) (width 0.5) (layer F.Cu) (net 6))
 (segment (start 181.2 121.92) (end 210.82 121.92) (width 0.5) (layer F.Cu) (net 6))
 (segment (start 176.022 114.2) (end 177.6505 115.8285) (width 0.5) (layer B.Cu) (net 6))
 (segment (start 177.6505 115.8285) (end 177.6505 116.9505) (width 0.5) (layer B.Cu) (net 6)))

